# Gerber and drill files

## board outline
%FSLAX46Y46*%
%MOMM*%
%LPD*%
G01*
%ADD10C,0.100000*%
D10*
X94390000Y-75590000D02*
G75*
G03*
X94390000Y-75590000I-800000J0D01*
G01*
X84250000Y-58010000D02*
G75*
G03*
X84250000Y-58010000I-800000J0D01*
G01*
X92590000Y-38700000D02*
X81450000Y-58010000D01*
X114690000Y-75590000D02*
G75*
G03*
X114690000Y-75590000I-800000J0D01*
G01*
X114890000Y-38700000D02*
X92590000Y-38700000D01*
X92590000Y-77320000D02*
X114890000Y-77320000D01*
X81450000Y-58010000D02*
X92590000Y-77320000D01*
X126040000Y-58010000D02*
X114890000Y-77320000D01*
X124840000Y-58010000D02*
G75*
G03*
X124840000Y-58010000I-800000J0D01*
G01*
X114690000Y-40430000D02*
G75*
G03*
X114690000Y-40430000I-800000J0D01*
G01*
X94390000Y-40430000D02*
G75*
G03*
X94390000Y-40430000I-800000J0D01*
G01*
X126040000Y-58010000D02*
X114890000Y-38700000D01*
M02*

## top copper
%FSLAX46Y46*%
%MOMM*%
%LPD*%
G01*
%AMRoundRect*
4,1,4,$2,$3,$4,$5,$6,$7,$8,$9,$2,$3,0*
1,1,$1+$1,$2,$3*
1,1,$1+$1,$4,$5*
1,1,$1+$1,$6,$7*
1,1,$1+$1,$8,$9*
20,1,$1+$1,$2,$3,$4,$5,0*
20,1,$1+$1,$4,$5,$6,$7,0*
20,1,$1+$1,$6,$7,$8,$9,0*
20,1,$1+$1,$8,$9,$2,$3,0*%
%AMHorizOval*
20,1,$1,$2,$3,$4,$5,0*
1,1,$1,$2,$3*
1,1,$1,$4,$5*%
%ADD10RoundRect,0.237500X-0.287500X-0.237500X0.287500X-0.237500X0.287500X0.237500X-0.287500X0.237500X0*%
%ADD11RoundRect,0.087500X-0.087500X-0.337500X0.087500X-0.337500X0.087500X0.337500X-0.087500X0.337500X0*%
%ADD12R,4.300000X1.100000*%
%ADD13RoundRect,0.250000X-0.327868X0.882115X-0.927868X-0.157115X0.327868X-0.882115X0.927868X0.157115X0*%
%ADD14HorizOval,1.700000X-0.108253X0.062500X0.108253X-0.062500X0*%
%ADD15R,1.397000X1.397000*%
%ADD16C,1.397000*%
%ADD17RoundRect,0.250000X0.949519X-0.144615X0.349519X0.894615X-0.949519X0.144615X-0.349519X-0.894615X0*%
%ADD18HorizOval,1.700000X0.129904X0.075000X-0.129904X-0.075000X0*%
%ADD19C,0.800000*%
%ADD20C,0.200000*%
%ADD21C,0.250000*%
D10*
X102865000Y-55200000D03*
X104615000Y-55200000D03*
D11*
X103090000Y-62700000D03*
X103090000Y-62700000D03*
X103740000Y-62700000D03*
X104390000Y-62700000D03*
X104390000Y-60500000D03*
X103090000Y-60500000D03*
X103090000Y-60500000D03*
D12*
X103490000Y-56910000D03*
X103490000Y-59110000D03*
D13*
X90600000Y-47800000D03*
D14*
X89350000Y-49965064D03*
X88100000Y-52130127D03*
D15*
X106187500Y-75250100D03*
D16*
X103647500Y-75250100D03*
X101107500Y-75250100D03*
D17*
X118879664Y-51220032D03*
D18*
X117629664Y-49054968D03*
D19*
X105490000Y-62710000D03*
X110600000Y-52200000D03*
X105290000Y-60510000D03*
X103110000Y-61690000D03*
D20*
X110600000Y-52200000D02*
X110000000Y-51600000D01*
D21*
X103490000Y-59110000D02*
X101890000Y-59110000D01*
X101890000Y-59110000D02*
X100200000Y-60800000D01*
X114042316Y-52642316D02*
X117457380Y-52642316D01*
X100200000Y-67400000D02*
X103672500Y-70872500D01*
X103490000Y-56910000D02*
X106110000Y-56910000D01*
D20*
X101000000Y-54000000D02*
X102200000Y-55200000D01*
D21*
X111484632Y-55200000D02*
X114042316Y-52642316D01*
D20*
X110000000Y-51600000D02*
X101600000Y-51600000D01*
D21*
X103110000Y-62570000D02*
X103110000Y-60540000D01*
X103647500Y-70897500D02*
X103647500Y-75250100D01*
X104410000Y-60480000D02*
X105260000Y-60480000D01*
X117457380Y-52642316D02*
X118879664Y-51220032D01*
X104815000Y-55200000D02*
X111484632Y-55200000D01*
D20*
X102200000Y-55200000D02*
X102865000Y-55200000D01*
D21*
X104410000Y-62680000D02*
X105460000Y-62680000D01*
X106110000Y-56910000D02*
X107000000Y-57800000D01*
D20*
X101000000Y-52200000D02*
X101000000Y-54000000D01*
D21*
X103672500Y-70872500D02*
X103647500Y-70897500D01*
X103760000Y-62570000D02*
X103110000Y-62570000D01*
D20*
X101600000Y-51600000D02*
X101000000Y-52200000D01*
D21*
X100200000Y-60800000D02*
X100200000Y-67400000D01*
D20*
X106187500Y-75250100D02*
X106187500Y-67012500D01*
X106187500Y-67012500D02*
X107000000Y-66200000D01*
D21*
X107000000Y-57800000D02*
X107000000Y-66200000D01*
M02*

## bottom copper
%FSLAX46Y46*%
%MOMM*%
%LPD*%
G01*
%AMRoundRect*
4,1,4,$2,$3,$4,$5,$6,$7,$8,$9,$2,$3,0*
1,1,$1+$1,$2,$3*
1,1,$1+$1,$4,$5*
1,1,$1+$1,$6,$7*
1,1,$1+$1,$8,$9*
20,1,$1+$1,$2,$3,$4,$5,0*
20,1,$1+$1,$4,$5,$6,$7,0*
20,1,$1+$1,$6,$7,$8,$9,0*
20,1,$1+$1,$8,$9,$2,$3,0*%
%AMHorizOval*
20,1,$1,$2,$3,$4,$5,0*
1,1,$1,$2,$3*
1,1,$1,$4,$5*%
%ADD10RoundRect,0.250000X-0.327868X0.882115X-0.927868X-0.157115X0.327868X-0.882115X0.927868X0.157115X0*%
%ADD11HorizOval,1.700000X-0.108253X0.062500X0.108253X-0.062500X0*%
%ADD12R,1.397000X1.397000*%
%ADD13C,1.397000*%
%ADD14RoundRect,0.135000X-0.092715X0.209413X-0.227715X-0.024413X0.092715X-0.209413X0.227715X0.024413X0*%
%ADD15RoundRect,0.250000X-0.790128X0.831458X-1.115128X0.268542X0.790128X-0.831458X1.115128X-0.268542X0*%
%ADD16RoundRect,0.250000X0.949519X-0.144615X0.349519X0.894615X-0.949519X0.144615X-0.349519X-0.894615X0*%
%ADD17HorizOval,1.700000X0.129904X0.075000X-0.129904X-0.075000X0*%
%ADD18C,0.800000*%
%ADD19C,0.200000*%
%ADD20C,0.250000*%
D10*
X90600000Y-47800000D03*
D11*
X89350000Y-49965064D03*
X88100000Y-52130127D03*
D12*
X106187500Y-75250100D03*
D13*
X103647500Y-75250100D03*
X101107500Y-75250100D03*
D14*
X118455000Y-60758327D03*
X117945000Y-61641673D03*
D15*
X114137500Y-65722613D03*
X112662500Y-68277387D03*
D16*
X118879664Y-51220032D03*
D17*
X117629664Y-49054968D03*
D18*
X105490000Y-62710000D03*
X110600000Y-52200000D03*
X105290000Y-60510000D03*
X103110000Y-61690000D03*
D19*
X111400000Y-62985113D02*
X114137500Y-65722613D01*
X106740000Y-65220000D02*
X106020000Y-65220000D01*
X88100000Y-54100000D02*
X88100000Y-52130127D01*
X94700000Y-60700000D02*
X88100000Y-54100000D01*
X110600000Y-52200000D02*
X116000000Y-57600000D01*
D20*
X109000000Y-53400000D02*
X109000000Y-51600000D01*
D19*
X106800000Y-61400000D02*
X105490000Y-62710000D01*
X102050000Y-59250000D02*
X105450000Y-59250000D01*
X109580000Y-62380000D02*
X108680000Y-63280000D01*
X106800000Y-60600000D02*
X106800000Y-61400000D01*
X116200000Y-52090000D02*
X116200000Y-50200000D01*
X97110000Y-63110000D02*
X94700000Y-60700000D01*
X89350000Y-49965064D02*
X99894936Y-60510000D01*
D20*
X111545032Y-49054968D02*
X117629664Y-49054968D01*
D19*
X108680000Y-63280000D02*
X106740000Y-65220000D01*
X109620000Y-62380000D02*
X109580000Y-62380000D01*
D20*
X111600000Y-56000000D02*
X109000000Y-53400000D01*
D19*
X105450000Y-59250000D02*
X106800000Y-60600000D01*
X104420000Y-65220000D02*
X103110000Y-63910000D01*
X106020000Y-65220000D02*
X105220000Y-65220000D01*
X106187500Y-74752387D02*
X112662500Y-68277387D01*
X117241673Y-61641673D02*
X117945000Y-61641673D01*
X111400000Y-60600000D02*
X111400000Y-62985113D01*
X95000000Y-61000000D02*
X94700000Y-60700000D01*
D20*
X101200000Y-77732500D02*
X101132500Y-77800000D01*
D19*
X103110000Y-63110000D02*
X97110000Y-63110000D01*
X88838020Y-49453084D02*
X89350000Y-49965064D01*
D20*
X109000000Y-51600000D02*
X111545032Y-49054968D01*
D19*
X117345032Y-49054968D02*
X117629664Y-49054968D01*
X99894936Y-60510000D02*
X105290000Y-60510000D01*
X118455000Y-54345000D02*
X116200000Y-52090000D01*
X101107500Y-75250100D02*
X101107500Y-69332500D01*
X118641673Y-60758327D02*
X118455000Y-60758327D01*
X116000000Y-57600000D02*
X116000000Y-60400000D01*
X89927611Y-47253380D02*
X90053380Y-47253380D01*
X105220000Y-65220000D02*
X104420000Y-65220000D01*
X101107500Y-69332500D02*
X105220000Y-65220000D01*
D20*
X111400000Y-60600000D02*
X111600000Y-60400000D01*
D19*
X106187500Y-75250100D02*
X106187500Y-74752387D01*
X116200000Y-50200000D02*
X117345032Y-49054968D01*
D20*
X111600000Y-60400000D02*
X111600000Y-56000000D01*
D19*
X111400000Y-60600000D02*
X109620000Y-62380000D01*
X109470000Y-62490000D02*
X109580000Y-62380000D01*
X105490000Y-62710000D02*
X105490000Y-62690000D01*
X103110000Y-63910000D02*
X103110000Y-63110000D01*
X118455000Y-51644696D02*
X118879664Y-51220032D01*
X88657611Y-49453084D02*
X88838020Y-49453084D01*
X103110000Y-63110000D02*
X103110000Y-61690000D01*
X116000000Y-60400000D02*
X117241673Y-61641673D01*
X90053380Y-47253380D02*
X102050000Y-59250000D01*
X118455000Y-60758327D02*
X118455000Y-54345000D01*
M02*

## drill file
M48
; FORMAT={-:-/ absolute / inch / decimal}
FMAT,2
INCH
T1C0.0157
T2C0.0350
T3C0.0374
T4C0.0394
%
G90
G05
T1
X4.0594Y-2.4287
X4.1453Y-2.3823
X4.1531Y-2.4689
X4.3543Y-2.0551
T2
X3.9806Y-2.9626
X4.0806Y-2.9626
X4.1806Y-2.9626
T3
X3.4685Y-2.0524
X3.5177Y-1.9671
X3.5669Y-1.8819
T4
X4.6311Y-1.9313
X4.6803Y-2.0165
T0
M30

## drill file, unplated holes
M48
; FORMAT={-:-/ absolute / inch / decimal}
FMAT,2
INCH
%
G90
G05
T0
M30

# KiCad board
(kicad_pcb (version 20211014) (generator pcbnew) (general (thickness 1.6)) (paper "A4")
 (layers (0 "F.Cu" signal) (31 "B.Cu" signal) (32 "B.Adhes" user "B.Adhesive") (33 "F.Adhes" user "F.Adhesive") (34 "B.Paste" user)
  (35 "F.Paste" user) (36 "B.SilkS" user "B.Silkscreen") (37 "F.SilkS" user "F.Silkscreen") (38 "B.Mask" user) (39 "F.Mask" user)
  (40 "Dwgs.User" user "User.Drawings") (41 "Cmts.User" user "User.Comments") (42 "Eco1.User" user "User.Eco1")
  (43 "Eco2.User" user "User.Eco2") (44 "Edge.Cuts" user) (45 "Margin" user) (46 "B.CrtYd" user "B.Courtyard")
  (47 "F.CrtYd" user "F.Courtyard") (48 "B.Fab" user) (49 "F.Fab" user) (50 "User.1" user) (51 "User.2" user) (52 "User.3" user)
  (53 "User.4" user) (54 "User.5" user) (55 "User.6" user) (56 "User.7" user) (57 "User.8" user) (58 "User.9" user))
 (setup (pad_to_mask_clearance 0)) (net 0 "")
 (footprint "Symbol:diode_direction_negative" (layer "F.Cu") (at 103.8 52.65)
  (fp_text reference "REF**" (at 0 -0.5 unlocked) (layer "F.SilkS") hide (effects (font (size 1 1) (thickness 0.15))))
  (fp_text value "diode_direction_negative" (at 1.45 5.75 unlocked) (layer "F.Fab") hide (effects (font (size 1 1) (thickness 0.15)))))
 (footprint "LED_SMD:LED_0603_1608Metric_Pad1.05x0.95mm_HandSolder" (layer "F.Cu") (at 103.74 55.2)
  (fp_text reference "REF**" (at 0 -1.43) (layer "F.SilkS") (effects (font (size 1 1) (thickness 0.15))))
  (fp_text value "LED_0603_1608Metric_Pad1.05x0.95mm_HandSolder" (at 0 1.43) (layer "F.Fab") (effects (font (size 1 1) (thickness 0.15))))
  (pad "1" smd roundrect (at -0.875 0) (size 1.05 0.95) (layers "F.Cu" "F.Paste" "F.Mask") (roundrect_rratio 0.25))
  (pad "2" smd roundrect (at 0.875 0) (size 1.05 0.95) (layers "F.Cu" "F.Paste" "F.Mask") (roundrect_rratio 0.25)))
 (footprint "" (layer "F.Cu") (at 103.09 62.7)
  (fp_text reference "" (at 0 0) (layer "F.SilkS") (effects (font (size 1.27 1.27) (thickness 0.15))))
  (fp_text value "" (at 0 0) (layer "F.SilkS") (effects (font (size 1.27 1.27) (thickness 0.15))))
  (pad "1" smd roundrect (at 0 0) (size 0.35 0.85) (layers "F.Cu" "F.Paste" "F.Mask") (roundrect_rratio 0.25)))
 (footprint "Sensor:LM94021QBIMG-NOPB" (layer "F.Cu") (at 103.74 61.6)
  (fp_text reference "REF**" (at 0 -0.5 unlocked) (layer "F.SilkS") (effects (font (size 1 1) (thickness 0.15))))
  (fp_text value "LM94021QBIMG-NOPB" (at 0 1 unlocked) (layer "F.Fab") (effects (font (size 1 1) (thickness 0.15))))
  (pad "1" smd roundrect (at -0.65 1.1) (size 0.35 0.85) (layers "F.Cu" "F.Paste" "F.Mask") (roundrect_rratio 0.25))
  (pad "2" smd roundrect (at 0 1.1) (size 0.35 0.85) (layers "F.Cu" "F.Paste" "F.Mask") (roundrect_rratio 0.25))
  (pad "3" smd roundrect (at 0.65 1.1) (size 0.35 0.85) (layers "F.Cu" "F.Paste" "F.Mask") (roundrect_rratio 0.25))
  (pad "4" smd roundrect (at 0.65 -1.1) (size 0.35 0.85) (layers "F.Cu" "F.Paste" "F.Mask") (roundrect_rratio 0.25))
  (pad "5" smd roundrect (at -0.65 -1.1) (size 0.35 0.85) (layers "F.Cu" "F.Paste" "F.Mask") (roundrect_rratio 0.25)))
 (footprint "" (layer "F.Cu") (at 103.09 60.5)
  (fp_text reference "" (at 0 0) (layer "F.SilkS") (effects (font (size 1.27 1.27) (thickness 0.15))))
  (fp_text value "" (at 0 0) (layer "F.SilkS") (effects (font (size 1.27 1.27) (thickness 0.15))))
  (pad "5" smd roundrect (at 0 0) (size 0.35 0.85) (layers "F.Cu" "F.Paste" "F.Mask") (roundrect_rratio 0.25)))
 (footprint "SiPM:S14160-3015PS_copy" (layer "F.Cu") (at 103.74 58.01)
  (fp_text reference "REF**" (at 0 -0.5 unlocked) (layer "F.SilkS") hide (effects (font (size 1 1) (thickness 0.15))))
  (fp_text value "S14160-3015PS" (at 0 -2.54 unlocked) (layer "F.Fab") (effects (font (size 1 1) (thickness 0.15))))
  (pad "1" smd rect (at -0.25 -1.1) (size 4.3 1.1) (layers "F.Cu" "F.Paste" "F.Mask"))
  (pad "2" smd rect (at -0.25 1.1) (size 4.3 1.1) (layers "F.Cu" "F.Paste" "F.Mask")))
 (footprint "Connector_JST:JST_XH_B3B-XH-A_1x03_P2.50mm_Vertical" (layer "B.Cu") (at 90.6 47.8 -120)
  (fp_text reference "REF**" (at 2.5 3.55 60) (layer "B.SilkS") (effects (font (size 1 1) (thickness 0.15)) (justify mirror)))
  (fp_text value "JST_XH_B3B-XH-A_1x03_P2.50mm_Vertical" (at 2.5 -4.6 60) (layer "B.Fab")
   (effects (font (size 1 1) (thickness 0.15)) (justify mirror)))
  (pad "1" thru_hole roundrect (at 0 0 240) (size 1.7 1.95) (drill 0.95) (layers *.Cu *.Mask) (roundrect_rratio 0.1470588235))
  (pad "2" thru_hole oval (at 2.5 0 240) (size 1.7 1.95) (drill 0.95) (layers *.Cu *.Mask))
  (pad "3" thru_hole oval (at 5 0 240) (size 1.7 1.95) (drill 0.95) (layers *.Cu *.Mask)))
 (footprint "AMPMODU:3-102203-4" (layer "B.Cu") (at 106.1875 75.2501 180)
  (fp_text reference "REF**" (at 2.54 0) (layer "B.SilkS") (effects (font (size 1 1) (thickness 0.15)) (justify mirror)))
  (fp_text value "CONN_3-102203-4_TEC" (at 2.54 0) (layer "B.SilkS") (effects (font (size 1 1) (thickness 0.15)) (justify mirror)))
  (pad "1" thru_hole rect locked (at 0 0 180) (size 1.397 1.397) (drill 0.889) (layers *.Cu *.Mask))
  (pad "2" thru_hole circle locked (at 2.54 0 180) (size 1.397 1.397) (drill 0.889) (layers *.Cu *.Mask))
  (pad "3" thru_hole circle locked (at 5.08 0 180) (size 1.397 1.397) (drill 0.889) (layers *.Cu *.Mask)))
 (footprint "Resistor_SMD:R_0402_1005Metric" (layer "B.Cu") (at 118.2 61.2 -120)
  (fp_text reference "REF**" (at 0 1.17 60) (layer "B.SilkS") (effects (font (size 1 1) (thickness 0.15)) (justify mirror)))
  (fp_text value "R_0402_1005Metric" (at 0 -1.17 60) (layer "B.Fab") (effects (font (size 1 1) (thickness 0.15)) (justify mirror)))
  (pad "1" smd roundrect (at -0.51 0 240) (size 0.54 0.64) (layers "B.Cu" "B.Paste" "B.Mask") (roundrect_rratio 0.25))
  (pad "2" smd roundrect (at 0.51 0 240) (size 0.54 0.64) (layers "B.Cu" "B.Paste" "B.Mask") (roundrect_rratio 0.25)))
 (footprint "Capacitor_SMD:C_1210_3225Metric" (layer "B.Cu") (at 113.4 67 -120)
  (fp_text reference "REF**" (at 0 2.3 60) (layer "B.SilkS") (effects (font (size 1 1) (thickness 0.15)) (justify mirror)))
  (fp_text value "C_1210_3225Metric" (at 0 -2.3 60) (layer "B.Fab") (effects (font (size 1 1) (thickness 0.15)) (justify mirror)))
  (pad "1" smd roundrect (at -1.475 0 240) (size 1.15 2.7) (layers "B.Cu" "B.Paste" "B.Mask") (roundrect_rratio 0.2173913043))
  (pad "2" smd roundrect (at 1.475 0 240) (size 1.15 2.7) (layers "B.Cu" "B.Paste" "B.Mask") (roundrect_rratio 0.2173913043)))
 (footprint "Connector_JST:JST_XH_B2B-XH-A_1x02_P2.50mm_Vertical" (layer "B.Cu") (at 118.879664 51.220032 120)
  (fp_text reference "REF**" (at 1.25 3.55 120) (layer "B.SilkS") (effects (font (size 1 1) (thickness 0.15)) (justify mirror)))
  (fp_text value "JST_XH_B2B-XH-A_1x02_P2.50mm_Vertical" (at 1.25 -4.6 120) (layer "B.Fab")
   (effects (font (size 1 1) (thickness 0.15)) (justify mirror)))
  (pad "1" thru_hole roundrect (at 0 0 120) (size 1.7 2) (drill 1) (layers *.Cu *.Mask) (roundrect_rratio 0.1470588235))
  (pad "2" thru_hole oval (at 2.5 0 120) (size 1.7 2) (drill 1) (layers *.Cu *.Mask)))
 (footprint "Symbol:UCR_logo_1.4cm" (layer "B.Cu") (at 104.4 43 180)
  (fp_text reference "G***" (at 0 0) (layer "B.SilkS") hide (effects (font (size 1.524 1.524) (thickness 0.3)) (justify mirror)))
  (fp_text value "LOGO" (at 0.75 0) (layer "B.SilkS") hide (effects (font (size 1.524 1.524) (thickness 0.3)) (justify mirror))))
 (gr_circle (center 93.59 75.59) (end 94.39 75.59) (layer "Edge.Cuts") (width 0.1) (fill none))
 (gr_circle (center 83.45 58.01) (end 84.25 58.01) (layer "Edge.Cuts") (width 0.1) (fill none))
 (gr_line (start 92.59 38.7) (end 81.45 58.01) (layer "Edge.Cuts") (width 0.1))
 (gr_circle (center 113.89 75.59) (end 114.69 75.59) (layer "Edge.Cuts") (width 0.1) (fill none))
 (gr_line (start 114.89 38.7) (end 92.59 38.7) (layer "Edge.Cuts") (width 0.1))
 (gr_line (start 92.59 77.32) (end 114.89 77.32) (layer "Edge.Cuts") (width 0.1))
 (gr_line (start 81.45 58.01) (end 92.59 77.32) (layer "Edge.Cuts") (width 0.1))
 (gr_line (start 126.04 58.01) (end 114.89 77.32) (layer "Edge.Cuts") (width 0.1))
 (gr_circle (center 124.04 58.01) (end 124.84 58.01) (layer "Edge.Cuts") (width 0.1) (fill none))
 (gr_circle (center 113.89 40.43) (end 114.69 40.43) (layer "Edge.Cuts") (width 0.1) (fill none))
 (gr_circle (center 93.59 40.43) (end 94.39 40.43) (layer "Edge.Cuts") (width 0.1) (fill none))
 (gr_line (start 126.04 58.01) (end 114.89 38.7) (layer "Edge.Cuts") (width 0.1))
 (segment (start 110.6 52.2) (end 110 51.6) (width 0.2) (layer "F.Cu") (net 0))
 (segment (start 103.49 59.11) (end 101.89 59.11) (width 0.25) (layer "F.Cu") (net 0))
 (segment (start 101.89 59.11) (end 100.2 60.8) (width 0.25) (layer "F.Cu") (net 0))
 (segment (start 114.042316 52.642316) (end 117.45738 52.642316) (width 0.25) (layer "F.Cu") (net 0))
 (segment (start 100.2 67.4) (end 103.6725 70.8725) (width 0.25) (layer "F.Cu") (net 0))
 (segment (start 103.49 56.91) (end 106.11 56.91) (width 0.25) (layer "F.Cu") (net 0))
 (segment (start 101 54) (end 102.2 55.2) (width 0.2) (layer "F.Cu") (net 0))
 (segment (start 111.484632 55.2) (end 114.042316 52.642316) (width 0.25) (layer "F.Cu") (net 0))
 (segment (start 110 51.6) (end 101.6 51.6) (width 0.2) (layer "F.Cu") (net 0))
 (segment (start 103.11 62.57) (end 103.11 60.54) (width 0.25) (layer "F.Cu") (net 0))
 (segment (start 103.6475 70.8975) (end 103.6475 75.2501) (width 0.25) (layer "F.Cu") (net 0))
 (segment (start 104.41 60.48) (end 105.26 60.48) (width 0.25) (layer "F.Cu") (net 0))
 (segment (start 117.45738 52.642316) (end 118.879664 51.220032) (width 0.25) (layer "F.Cu") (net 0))
 (segment (start 104.815 55.2) (end 111.484632 55.2) (width 0.25) (layer "F.Cu") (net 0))
 (segment (start 102.2 55.2) (end 102.865 55.2) (width 0.2) (layer "F.Cu") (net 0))
 (segment (start 104.41 62.68) (end 105.46 62.68) (width 0.25) (layer "F.Cu") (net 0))
 (segment (start 106.11 56.91) (end 107 57.8) (width 0.25) (layer "F.Cu") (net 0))
 (segment (start 101 52.2) (end 101 54) (width 0.2) (layer "F.Cu") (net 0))
 (segment (start 103.6725 70.8725) (end 103.6475 70.8975) (width 0.25) (layer "F.Cu") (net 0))
 (segment (start 103.76 62.57) (end 103.11 62.57) (width 0.25) (layer "F.Cu") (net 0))
 (segment (start 101.6 51.6) (end 101 52.2) (width 0.2) (layer "F.Cu") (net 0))
 (segment (start 100.2 60.8) (end 100.2 67.4) (width 0.25) (layer "F.Cu") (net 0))
 (segment (start 106.1875 75.2501) (end 106.1875 67.0125) (width 0.2) (layer "F.Cu") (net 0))
 (segment (start 106.1875 67.0125) (end 107 66.2) (width 0.2) (layer "F.Cu") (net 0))
 (segment (start 107 57.8) (end 107 66.2) (width 0.25) (layer "F.Cu") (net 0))
 (via (at 105.49 62.71) (size 0.8) (drill 0.4) (layers "F.Cu" "B.Cu") (free) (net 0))
 (via (at 110.6 52.2) (size 0.8) (drill 0.4) (layers "F.Cu" "B.Cu") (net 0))
 (via (at 105.29 60.51) (size 0.8) (drill 0.4) (layers "F.Cu" "B.Cu") (free) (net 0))
 (via (at 103.11 61.69) (size 0.8) (drill 0.4) (layers "F.Cu" "B.Cu") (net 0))
 (segment (start 111.4 62.985113) (end 114.1375 65.722613) (width 0.2) (layer "B.Cu") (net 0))
 (segment (start 106.74 65.22) (end 106.02 65.22) (width 0.2) (layer "B.Cu") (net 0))
 (segment (start 88.1 54.1) (end 88.1 52.130127) (width 0.2) (layer "B.Cu") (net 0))
 (segment (start 94.7 60.7) (end 88.1 54.1) (width 0.2) (layer "B.Cu") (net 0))
 (segment (start 110.6 52.2) (end 116 57.6) (width 0.2) (layer "B.Cu") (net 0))
 (segment (start 109 53.4) (end 109 51.6) (width 0.25) (layer "B.Cu") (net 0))
 (segment (start 106.8 61.4) (end 105.49 62.71) (width 0.2) (layer "B.Cu") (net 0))
 (segment (start 102.05 59.25) (end 105.45 59.25) (width 0.2) (layer "B.Cu") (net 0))
 (segment (start 109.58 62.38) (end 108.68 63.28) (width 0.2) (layer "B.Cu") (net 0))
 (segment (start 106.8 60.6) (end 106.8 61.4) (width 0.2) (layer "B.Cu") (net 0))
 (segment (start 116.2 52.09) (end 116.2 50.2) (width 0.2) (layer "B.Cu") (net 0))
 (segment (start 97.11 63.11) (end 94.7 60.7) (width 0.2) (layer "B.Cu") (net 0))
 (segment (start 89.35 49.965064) (end 99.894936 60.51) (width 0.2) (layer "B.Cu") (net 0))
 (segment (start 111.545032 49.054968) (end 117.629664 49.054968) (width 0.25) (layer "B.Cu") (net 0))
 (segment (start 108.68 63.28) (end 106.74 65.22) (width 0.2) (layer "B.Cu") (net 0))
 (segment (start 109.62 62.38) (end 109.58 62.38) (width 0.2) (layer "B.Cu") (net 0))
 (segment (start 111.6 56) (end 109 53.4) (width 0.25) (layer "B.Cu") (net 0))
 (segment (start 105.45 59.25) (end 106.8 60.6) (width 0.2) (layer "B.Cu") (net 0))
 (segment (start 104.42 65.22) (end 103.11 63.91) (width 0.2) (layer "B.Cu") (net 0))
 (segment (start 106.02 65.22) (end 105.22 65.22) (width 0.2) (layer "B.Cu") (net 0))
 (segment (start 106.1875 74.752387) (end 112.6625 68.277387) (width 0.2) (layer "B.Cu") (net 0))
 (segment (start 117.241673 61.641673) (end 117.945 61.641673) (width 0.2) (layer "B.Cu") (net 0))
 (segment (start 111.4 60.6) (end 111.4 62.985113) (width 0.2) (layer "B.Cu") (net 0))
 (segment (start 95 61) (end 94.7 60.7) (width 0.2) (layer "B.Cu") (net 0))
 (segment (start 101.2 77.7325) (end 101.1325 77.8) (width 0.25) (layer "B.Cu") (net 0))
 (segment (start 103.11 63.11) (end 97.11 63.11) (width 0.2) (layer "B.Cu") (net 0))
 (segment (start 88.83802 49.453084) (end 89.35 49.965064) (width 0.2) (layer "B.Cu") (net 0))
 (segment (start 109 51.6) (end 111.545032 49.054968) (width 0.25) (layer "B.Cu") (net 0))
 (segment (start 117.345032 49.054968) (end 117.629664 49.054968) (width 0.2) (layer "B.Cu") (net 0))
 (segment (start 99.894936 60.51) (end 105.29 60.51) (width 0.2) (layer "B.Cu") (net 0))
 (segment (start 118.455 54.345) (end 116.2 52.09) (width 0.2) (layer "B.Cu") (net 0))
 (segment (start 101.1075 75.2501) (end 101.1075 69.3325) (width 0.2) (layer "B.Cu") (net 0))
 (segment (start 118.641673 60.758327) (end 118.455 60.758327) (width 0.2) (layer "B.Cu") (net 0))
 (segment (start 116 57.6) (end 116 60.4) (width 0.2) (layer "B.Cu") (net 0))
 (segment (start 89.927611 47.25338) (end 90.05338 47.25338) (width 0.2) (layer "B.Cu") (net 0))
 (segment (start 105.22 65.22) (end 104.42 65.22) (width 0.2) (layer "B.Cu") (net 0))
 (segment (start 101.1075 69.3325) (end 105.22 65.22) (width 0.2) (layer "B.Cu") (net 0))
 (segment (start 111.4 60.6) (end 111.6 60.4) (width 0.25) (layer "B.Cu") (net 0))
 (segment (start 106.1875 75.2501) (end 106.1875 74.752387) (width 0.2) (layer "B.Cu") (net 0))
 (segment (start 116.2 50.2) (end 117.345032 49.054968) (width 0.2) (layer "B.Cu") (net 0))
 (segment (start 111.6 60.4) (end 111.6 56) (width 0.25) (layer "B.Cu") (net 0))
 (segment (start 111.4 60.6) (end 109.62 62.38) (width 0.2) (layer "B.Cu") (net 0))
 (segment (start 109.47 62.49) (end 109.58 62.38) (width 0.2) (layer "B.Cu") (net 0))
 (segment (start 105.49 62.71) (end 105.49 62.69) (width 0.2) (layer "B.Cu") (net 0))
 (segment (start 103.11 63.91) (end 103.11 63.11) (width 0.2) (layer "B.Cu") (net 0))
 (segment (start 118.455 51.644696) (end 118.879664 51.220032) (width 0.2) (layer "B.Cu") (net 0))
 (segment (start 88.657611 49.453084) (end 88.83802 49.453084) (width 0.2) (layer "B.Cu") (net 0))
 (segment (start 103.11 63.11) (end 103.11 61.69) (width 0.2) (layer "B.Cu") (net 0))
 (segment (start 116 60.4) (end 117.241673 61.641673) (width 0.2) (layer "B.Cu") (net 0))
 (segment (start 90.05338 47.25338) (end 102.05 59.25) (width 0.2) (layer "B.Cu") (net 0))
 (segment (start 118.455 60.758327) (end 118.455 54.345) (width 0.2) (layer "B.Cu") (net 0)))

